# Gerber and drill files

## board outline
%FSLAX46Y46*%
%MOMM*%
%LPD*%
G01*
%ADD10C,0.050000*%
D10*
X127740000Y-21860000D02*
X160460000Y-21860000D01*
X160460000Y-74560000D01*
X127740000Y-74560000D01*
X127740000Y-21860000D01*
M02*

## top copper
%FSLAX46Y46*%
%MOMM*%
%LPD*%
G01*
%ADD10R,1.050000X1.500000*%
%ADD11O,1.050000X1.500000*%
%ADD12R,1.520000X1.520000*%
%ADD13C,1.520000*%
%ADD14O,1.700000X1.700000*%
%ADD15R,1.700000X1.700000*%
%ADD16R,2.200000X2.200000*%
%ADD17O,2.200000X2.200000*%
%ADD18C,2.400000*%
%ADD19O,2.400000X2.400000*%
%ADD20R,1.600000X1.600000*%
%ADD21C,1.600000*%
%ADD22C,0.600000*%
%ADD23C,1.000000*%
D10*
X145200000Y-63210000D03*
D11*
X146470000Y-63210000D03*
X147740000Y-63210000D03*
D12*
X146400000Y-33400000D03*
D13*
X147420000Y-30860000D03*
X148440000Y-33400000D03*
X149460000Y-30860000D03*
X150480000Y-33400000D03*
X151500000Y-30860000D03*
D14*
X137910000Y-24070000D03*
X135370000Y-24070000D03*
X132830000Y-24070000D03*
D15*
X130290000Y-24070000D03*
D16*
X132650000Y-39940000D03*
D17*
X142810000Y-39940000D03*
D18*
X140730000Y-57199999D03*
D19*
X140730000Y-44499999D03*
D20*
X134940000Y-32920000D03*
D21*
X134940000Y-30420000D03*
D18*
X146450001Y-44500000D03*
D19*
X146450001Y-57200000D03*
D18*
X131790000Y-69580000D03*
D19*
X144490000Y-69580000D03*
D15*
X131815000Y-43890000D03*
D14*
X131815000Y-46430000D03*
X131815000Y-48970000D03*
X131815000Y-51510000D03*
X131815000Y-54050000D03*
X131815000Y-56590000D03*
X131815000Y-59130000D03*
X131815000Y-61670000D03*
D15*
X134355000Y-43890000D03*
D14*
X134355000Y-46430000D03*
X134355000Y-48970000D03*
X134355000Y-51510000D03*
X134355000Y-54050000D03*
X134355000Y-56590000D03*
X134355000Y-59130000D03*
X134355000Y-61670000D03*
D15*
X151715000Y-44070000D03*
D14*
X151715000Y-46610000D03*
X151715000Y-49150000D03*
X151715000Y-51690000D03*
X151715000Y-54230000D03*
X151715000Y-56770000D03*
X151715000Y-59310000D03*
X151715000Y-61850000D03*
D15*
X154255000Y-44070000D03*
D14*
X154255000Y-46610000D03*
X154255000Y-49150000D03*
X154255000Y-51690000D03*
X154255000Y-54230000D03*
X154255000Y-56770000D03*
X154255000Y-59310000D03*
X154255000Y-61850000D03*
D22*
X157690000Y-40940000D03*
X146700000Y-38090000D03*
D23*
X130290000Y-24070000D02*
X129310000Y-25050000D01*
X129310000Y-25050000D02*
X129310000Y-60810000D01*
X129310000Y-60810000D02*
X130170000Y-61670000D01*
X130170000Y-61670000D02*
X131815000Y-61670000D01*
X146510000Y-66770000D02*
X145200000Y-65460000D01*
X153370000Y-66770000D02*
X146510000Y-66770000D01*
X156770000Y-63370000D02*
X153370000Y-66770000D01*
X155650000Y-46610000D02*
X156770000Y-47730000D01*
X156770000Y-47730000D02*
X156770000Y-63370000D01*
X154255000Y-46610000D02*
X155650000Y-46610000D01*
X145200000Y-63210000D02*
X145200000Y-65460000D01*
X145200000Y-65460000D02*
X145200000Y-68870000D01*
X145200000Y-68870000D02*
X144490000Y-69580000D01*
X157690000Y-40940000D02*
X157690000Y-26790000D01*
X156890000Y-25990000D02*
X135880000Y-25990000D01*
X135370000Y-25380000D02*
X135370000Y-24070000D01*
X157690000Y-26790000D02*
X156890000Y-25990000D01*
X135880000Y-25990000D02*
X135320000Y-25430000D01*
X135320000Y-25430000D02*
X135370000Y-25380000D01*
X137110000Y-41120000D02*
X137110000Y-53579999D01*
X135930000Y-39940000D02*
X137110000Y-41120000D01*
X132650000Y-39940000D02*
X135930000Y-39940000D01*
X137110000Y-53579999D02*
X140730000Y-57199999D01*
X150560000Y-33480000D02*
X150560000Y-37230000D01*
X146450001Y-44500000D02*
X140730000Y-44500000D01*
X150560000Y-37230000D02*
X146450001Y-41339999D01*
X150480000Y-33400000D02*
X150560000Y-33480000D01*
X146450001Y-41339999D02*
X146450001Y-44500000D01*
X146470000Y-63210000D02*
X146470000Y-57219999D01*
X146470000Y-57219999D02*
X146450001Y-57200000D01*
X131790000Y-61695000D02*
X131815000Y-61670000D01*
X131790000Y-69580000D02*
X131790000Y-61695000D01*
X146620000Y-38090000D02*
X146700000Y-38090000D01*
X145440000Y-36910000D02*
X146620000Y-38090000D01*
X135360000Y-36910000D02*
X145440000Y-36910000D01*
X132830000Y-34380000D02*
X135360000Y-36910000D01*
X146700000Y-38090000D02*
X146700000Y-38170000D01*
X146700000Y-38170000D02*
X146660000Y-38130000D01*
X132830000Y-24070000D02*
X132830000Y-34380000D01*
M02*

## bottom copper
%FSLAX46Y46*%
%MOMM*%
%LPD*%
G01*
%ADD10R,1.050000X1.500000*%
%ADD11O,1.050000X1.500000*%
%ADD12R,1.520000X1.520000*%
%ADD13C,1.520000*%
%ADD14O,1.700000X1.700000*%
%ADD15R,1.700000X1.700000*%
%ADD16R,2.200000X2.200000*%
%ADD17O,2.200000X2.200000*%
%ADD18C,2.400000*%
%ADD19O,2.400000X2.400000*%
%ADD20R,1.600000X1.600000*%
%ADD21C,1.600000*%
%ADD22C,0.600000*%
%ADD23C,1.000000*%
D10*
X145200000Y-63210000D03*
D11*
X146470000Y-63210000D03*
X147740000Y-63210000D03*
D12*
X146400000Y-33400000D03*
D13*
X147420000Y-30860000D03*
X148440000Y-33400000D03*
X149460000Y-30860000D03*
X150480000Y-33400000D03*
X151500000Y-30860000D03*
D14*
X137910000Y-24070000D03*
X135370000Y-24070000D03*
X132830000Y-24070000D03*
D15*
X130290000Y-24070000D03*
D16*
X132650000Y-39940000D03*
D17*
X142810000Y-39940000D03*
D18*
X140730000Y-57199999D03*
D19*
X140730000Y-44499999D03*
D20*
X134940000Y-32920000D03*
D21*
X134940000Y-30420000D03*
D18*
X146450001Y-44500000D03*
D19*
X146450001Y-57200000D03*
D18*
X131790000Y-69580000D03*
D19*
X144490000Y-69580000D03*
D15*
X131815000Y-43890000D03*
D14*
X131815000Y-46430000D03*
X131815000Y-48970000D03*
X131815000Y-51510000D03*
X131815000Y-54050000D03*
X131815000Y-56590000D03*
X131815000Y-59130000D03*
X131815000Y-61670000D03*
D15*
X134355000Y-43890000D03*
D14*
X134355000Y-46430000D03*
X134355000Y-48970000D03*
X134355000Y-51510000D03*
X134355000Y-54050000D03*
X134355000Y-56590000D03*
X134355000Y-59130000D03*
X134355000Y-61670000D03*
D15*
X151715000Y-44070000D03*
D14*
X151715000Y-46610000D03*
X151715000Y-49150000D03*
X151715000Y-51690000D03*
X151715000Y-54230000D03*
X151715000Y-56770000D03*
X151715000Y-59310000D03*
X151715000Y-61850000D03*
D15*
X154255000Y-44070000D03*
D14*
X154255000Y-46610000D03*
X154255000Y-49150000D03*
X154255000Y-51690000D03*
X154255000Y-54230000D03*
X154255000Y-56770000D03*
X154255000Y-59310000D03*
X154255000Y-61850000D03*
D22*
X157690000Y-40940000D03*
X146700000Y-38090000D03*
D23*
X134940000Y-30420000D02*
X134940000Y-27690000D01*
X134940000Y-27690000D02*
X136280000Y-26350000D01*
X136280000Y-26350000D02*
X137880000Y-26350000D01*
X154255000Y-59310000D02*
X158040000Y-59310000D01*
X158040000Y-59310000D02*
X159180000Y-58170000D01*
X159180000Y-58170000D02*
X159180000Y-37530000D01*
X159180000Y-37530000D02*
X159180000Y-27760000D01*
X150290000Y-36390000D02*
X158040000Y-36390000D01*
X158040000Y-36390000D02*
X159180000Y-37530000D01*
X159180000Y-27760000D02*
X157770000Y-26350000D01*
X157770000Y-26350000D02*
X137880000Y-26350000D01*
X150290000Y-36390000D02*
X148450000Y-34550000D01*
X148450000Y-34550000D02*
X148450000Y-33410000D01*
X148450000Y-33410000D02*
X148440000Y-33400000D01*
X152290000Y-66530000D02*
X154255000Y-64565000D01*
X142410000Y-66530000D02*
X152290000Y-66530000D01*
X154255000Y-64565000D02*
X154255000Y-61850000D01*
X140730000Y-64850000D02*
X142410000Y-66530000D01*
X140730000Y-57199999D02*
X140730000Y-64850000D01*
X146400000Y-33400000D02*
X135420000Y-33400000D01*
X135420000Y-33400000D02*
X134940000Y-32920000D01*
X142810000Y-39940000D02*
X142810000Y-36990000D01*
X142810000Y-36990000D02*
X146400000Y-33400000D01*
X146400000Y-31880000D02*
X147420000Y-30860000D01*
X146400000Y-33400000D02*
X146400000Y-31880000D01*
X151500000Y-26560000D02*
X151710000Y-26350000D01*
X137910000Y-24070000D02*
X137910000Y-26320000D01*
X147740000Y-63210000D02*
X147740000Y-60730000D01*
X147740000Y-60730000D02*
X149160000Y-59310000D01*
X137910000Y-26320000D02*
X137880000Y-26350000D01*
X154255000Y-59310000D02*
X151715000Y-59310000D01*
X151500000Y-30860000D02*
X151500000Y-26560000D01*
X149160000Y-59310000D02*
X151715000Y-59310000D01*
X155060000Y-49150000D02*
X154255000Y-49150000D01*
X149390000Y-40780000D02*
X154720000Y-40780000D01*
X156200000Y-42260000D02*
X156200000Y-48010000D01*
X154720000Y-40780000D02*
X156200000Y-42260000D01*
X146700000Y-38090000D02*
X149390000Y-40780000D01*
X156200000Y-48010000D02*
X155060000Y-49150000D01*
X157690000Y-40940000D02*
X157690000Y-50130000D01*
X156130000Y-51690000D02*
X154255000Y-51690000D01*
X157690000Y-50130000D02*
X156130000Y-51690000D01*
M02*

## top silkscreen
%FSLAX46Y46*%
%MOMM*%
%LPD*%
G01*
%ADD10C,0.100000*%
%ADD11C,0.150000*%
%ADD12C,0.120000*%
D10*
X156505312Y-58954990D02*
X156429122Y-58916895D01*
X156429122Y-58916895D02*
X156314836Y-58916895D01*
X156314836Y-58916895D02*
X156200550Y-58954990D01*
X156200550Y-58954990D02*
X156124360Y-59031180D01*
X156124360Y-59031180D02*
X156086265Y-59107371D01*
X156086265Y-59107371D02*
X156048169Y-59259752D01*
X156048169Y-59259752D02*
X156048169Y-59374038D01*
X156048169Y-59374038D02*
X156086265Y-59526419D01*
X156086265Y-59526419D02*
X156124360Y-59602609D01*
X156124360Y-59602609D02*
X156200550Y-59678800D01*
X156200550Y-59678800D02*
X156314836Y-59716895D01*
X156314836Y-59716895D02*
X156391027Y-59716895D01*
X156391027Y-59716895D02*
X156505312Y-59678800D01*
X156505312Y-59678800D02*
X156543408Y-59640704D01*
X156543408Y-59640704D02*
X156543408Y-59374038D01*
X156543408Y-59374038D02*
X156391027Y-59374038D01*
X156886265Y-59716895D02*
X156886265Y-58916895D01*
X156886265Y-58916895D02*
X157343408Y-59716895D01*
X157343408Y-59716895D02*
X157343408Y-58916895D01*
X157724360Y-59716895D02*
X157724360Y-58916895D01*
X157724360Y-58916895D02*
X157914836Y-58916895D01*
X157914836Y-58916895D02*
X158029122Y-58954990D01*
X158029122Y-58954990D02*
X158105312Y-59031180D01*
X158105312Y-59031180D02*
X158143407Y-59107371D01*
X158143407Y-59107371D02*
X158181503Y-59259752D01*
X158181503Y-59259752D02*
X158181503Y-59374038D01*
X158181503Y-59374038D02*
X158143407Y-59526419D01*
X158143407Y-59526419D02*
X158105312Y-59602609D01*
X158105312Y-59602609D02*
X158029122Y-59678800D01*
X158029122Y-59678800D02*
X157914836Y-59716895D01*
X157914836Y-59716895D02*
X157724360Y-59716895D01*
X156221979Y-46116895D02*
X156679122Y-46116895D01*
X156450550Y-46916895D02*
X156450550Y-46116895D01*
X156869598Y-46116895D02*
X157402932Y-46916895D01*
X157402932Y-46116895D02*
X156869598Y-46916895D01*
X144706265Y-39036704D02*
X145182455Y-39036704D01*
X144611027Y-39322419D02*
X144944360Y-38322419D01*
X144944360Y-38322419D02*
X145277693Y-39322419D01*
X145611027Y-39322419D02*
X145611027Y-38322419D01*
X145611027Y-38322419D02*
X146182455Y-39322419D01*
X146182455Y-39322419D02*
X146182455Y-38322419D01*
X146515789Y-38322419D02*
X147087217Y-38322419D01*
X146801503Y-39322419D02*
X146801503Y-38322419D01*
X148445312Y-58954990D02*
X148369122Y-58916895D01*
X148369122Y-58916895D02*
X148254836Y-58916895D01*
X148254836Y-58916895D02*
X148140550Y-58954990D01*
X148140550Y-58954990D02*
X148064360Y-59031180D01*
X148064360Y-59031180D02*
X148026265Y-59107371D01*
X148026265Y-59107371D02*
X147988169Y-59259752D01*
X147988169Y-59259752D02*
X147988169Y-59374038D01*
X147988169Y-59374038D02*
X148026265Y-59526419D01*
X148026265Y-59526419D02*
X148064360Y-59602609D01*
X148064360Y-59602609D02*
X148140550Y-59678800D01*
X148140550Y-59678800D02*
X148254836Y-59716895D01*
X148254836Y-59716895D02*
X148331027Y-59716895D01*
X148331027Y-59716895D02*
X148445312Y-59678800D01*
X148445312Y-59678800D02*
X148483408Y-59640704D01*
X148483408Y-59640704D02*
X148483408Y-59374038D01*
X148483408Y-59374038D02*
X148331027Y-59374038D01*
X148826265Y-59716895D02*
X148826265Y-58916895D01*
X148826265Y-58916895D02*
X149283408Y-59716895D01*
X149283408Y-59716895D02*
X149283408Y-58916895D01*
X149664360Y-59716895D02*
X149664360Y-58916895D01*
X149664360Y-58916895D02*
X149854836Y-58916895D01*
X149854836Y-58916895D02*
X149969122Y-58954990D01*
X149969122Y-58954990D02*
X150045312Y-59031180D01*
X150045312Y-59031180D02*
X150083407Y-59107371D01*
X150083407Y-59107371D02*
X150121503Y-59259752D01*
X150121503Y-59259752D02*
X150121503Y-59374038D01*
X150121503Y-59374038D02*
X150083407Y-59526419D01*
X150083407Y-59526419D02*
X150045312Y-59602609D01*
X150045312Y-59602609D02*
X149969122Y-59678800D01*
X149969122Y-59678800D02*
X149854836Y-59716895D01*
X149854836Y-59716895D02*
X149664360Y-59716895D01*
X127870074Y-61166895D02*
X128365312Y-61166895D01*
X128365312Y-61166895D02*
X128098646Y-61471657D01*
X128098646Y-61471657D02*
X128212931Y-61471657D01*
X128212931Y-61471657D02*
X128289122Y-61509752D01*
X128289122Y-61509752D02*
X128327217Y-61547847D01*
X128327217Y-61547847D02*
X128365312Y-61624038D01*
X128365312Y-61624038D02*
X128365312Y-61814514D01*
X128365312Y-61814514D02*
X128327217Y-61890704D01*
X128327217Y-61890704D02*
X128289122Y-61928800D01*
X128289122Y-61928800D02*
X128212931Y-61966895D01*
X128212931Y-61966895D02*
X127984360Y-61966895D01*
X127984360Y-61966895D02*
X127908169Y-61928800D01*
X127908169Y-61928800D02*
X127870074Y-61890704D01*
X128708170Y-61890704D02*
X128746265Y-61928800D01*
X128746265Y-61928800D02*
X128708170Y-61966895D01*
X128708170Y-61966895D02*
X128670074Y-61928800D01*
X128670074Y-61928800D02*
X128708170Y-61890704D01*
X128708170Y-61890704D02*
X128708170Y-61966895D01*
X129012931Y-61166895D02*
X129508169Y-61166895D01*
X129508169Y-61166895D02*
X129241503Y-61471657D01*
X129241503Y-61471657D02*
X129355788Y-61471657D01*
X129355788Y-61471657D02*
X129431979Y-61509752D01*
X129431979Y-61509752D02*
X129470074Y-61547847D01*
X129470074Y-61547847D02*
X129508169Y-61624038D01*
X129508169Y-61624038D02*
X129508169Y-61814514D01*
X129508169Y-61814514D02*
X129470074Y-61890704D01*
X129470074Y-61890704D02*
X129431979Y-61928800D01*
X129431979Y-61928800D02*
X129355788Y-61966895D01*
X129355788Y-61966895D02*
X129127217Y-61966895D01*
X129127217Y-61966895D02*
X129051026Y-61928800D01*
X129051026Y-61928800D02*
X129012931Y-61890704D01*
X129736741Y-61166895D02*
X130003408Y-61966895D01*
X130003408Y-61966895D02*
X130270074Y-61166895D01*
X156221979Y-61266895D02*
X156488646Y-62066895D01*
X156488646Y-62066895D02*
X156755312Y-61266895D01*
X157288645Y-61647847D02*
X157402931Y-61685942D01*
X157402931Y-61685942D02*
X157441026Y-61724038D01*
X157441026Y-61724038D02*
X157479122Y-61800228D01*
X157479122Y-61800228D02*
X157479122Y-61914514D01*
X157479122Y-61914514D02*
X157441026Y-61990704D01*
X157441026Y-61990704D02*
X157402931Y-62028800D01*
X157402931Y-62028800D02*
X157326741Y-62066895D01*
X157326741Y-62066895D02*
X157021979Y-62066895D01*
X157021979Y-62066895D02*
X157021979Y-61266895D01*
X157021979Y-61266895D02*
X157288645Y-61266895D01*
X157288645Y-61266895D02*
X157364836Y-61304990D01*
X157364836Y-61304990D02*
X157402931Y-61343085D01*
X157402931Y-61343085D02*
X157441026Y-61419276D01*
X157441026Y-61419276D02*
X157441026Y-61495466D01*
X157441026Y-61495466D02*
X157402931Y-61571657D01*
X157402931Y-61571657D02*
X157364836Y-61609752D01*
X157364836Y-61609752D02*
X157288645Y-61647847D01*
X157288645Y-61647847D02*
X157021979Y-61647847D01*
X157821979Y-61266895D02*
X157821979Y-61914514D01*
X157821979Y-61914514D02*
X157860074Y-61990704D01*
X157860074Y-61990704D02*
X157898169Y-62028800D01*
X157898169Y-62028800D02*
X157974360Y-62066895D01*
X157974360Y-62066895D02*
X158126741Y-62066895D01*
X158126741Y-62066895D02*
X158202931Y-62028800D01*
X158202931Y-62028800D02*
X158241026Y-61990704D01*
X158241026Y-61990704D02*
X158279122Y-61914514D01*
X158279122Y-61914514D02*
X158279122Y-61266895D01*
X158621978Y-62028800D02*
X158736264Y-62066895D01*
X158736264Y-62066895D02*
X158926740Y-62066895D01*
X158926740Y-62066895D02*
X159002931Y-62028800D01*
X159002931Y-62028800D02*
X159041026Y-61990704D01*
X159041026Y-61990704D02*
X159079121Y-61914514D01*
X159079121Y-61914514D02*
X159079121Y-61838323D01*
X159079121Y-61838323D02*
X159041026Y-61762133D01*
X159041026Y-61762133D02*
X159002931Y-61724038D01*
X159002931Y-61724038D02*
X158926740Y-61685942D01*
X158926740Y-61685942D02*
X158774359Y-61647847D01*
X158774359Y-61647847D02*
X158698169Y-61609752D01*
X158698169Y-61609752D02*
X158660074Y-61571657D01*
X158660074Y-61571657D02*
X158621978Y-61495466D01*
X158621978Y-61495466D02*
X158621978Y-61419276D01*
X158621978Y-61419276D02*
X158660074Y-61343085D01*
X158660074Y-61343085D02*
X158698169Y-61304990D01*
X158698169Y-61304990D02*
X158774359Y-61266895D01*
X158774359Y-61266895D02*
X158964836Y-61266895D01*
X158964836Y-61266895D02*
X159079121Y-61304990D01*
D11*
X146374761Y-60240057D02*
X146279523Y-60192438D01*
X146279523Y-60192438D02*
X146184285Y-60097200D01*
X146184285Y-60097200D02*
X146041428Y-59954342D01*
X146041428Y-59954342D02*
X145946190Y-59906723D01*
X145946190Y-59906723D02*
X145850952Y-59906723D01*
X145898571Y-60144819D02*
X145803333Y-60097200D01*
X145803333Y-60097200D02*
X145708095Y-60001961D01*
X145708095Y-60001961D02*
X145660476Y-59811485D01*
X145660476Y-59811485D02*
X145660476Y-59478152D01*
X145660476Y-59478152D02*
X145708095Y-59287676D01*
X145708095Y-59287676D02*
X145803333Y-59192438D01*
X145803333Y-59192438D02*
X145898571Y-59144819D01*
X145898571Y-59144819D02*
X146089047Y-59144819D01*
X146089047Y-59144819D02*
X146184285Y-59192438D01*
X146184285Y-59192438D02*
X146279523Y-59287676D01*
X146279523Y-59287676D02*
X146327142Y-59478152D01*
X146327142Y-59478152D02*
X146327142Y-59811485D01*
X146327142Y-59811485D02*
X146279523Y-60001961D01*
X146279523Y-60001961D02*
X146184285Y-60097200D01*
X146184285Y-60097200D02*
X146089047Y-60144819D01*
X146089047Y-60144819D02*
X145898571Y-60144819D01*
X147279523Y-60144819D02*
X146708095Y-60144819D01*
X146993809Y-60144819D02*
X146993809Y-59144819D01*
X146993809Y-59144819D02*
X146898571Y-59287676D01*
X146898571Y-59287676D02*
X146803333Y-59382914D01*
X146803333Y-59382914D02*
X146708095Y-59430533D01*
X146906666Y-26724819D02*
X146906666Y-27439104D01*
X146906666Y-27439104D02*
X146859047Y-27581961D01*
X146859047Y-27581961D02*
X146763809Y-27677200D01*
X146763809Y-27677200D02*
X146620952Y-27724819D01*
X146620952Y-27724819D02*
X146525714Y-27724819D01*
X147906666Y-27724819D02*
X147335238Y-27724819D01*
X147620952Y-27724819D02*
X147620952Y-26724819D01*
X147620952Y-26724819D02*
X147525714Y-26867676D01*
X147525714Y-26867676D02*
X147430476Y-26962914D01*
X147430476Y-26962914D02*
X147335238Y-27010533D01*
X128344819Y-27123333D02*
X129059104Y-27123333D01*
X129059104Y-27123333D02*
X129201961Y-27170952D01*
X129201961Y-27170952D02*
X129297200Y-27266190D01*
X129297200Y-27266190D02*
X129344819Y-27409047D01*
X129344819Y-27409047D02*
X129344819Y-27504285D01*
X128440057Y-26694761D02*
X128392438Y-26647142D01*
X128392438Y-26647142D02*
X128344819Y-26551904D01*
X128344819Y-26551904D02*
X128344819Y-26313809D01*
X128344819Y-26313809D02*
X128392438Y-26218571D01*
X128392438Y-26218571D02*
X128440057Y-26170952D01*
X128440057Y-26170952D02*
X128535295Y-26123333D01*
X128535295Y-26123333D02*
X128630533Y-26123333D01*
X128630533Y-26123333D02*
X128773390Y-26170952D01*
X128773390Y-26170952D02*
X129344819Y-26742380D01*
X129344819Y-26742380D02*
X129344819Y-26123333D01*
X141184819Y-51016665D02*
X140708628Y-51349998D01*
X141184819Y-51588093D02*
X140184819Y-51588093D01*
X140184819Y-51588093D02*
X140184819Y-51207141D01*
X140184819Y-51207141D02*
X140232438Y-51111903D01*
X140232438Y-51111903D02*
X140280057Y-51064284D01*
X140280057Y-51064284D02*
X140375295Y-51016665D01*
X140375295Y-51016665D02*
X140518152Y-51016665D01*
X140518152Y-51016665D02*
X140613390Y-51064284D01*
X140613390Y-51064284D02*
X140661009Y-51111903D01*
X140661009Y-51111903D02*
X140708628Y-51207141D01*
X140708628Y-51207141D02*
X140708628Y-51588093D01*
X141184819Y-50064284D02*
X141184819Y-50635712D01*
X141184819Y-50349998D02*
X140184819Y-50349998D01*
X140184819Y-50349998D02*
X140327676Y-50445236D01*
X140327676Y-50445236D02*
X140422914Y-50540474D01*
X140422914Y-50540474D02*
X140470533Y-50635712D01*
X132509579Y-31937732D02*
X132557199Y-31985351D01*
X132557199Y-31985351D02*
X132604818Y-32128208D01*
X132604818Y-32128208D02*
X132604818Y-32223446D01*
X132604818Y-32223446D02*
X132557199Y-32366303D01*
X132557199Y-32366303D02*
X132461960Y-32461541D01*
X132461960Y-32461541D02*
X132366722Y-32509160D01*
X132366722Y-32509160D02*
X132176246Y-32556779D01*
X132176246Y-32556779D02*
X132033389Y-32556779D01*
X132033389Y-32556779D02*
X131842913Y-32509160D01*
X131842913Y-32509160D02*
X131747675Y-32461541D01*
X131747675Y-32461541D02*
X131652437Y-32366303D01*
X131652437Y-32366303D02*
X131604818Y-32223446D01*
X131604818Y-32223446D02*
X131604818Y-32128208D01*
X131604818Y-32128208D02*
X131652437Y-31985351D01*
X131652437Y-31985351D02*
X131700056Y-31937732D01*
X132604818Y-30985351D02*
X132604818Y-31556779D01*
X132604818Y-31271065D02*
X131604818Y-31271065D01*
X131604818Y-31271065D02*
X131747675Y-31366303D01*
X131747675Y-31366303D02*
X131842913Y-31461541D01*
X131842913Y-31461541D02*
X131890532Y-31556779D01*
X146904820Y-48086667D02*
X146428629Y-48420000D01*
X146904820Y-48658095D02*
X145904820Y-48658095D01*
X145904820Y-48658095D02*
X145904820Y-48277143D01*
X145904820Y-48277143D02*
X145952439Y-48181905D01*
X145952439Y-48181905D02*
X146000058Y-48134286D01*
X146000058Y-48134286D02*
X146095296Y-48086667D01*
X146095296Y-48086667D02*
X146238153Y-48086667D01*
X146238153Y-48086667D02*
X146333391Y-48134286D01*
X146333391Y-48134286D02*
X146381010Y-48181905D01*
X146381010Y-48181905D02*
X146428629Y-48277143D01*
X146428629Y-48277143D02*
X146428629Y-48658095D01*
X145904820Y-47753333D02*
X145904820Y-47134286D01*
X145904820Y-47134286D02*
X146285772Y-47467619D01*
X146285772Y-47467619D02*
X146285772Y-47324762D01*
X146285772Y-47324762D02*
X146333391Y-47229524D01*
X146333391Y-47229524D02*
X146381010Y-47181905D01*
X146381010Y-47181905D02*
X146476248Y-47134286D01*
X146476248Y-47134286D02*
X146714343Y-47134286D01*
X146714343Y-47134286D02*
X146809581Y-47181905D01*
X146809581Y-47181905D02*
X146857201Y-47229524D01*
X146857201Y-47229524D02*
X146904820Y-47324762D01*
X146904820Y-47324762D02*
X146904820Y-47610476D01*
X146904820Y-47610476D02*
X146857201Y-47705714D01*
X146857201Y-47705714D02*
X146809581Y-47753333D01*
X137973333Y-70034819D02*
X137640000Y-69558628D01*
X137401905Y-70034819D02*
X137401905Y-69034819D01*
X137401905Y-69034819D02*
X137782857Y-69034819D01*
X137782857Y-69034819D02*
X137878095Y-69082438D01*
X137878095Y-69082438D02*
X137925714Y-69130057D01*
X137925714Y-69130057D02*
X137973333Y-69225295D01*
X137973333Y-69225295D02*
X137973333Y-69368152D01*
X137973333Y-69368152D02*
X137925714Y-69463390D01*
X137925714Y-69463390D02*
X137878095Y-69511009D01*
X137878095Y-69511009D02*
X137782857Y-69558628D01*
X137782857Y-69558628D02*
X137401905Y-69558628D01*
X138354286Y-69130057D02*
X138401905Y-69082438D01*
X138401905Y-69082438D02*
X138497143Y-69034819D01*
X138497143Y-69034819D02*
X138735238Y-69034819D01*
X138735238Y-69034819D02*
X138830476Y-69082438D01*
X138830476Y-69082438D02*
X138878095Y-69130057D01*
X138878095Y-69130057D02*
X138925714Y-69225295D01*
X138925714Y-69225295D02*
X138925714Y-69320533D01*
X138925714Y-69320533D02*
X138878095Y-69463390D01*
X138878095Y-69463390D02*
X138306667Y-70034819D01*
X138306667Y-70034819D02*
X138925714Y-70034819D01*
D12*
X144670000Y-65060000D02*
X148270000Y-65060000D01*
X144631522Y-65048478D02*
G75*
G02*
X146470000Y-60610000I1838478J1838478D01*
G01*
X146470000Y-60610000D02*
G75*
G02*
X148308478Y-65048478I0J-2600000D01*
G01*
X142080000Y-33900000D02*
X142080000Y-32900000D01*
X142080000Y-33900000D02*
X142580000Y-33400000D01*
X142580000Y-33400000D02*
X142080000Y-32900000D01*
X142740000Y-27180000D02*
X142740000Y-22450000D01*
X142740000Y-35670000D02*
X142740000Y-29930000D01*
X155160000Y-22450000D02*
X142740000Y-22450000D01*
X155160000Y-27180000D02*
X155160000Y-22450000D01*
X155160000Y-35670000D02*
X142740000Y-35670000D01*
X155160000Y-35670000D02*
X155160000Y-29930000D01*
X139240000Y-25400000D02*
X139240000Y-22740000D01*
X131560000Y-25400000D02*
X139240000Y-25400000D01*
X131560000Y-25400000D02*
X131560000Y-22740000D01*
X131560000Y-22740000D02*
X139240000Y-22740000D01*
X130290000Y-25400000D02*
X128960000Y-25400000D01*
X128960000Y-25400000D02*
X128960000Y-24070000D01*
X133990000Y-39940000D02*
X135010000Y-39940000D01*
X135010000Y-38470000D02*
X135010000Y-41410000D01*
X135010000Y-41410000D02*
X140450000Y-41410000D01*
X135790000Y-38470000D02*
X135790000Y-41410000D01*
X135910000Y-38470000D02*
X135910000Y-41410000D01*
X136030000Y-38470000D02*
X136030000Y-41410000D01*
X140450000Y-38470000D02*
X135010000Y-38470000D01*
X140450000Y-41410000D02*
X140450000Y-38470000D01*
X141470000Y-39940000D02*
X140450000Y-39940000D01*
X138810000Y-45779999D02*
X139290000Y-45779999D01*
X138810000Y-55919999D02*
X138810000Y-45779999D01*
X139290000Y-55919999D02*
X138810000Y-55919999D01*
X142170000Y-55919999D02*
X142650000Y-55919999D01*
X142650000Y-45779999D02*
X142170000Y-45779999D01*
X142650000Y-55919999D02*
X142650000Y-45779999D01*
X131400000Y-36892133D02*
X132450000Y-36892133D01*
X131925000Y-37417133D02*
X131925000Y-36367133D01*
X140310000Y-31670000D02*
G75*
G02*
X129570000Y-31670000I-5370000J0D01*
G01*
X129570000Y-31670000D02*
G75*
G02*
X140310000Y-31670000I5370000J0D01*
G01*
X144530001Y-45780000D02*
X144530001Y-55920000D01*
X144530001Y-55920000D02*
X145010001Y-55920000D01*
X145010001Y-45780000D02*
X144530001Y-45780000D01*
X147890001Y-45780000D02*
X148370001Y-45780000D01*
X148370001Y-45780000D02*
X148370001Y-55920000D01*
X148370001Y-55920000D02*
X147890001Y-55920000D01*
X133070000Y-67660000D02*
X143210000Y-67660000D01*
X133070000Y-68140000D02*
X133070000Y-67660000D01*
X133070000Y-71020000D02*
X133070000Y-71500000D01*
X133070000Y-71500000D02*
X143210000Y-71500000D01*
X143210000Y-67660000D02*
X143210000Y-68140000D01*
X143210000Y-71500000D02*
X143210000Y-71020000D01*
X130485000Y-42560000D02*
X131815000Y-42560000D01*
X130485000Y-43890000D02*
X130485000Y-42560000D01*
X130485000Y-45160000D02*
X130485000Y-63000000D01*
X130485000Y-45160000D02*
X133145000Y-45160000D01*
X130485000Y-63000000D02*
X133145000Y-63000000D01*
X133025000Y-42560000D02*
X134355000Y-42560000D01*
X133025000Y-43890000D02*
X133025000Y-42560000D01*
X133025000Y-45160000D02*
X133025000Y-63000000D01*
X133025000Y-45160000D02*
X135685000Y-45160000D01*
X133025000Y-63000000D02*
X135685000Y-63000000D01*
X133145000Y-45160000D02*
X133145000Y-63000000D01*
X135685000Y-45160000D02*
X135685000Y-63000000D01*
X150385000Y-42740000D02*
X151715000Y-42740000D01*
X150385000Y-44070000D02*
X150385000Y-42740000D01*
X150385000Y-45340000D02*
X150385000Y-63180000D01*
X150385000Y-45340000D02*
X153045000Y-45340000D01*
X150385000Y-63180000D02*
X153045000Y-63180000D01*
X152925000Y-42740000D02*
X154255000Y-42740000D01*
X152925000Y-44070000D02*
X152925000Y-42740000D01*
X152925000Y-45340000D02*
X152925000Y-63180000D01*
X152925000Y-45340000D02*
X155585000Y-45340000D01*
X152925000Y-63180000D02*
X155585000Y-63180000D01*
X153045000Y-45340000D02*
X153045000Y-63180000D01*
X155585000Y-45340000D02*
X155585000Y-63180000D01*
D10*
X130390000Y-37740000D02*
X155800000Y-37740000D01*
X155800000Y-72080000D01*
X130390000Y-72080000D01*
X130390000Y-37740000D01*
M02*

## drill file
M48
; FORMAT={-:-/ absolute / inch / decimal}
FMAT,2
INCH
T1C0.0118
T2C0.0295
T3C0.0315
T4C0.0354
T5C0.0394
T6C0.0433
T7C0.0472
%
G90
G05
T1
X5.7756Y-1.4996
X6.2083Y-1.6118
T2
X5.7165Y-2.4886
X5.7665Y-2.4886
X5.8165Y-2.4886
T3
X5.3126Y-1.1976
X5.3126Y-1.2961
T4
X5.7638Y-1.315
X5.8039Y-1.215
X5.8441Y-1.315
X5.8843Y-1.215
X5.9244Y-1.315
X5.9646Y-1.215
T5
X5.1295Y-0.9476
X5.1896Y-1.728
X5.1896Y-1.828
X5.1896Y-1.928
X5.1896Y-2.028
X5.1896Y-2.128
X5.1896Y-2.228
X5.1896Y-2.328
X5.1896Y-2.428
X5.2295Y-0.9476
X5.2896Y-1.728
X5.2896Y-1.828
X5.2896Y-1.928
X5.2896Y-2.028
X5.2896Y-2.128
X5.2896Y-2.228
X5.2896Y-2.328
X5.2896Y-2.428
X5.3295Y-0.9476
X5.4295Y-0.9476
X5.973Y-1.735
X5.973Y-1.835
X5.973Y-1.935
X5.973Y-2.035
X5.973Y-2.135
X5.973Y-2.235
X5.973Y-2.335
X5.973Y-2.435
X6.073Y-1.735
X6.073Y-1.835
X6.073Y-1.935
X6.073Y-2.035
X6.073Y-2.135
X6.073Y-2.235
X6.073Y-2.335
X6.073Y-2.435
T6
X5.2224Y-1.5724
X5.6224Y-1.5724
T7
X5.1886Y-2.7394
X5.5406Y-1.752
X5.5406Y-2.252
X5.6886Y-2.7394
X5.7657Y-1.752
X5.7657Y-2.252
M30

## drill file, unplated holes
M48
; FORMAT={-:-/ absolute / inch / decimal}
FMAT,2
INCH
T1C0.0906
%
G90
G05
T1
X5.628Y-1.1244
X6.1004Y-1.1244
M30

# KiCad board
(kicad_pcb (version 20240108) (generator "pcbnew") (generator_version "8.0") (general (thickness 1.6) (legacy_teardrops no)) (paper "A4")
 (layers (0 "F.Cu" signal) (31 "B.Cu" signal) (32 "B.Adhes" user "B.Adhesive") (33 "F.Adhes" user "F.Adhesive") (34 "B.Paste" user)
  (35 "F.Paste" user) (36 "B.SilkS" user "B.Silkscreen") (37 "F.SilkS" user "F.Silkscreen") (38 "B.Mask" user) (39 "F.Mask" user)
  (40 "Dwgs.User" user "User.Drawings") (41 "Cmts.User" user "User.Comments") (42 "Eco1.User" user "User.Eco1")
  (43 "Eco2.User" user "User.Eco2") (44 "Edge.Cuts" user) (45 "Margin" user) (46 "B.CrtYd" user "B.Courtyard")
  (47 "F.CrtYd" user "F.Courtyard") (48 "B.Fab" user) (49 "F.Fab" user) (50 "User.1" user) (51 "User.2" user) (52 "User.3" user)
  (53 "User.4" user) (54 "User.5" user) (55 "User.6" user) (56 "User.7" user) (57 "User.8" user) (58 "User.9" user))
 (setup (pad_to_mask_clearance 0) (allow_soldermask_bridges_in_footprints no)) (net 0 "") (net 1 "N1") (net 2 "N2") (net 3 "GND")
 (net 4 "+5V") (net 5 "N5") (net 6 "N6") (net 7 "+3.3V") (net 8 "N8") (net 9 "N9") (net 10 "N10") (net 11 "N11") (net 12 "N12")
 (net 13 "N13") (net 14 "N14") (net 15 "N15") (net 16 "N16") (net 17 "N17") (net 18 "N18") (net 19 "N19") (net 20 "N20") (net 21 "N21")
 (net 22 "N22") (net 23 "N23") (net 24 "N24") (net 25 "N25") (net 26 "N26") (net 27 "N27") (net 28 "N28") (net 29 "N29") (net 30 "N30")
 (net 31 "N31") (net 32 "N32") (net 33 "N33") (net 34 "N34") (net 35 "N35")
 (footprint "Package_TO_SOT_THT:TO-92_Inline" (layer "F.Cu") (at 145.2 63.21)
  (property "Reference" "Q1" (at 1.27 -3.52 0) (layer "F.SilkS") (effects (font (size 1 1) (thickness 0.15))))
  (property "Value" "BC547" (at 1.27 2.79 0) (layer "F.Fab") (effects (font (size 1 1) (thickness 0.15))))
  (fp_line (start -0.53 1.85) (end 3.07 1.85) (stroke (width 0.12) (type solid)) (layer "F.SilkS"))
  (fp_arc (start -0.568478 1.838478) (mid -1.132087 -0.994977) (end 1.27 -2.6) (stroke (width 0.12) (type solid)) (layer "F.SilkS"))
  (fp_arc (start 1.27 -2.6) (mid 3.672087 -0.994977) (end 3.108478 1.838478) (stroke (width 0.12) (type solid)) (layer "F.SilkS"))
  (pad "1" thru_hole rect (at 0 0) (size 1.05 1.5) (drill 0.75) (layers "*.Cu" "*.Mask") (remove_unused_layers no) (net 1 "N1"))
  (pad "2" thru_hole oval (at 1.27 0) (size 1.05 1.5) (drill 0.75) (layers "*.Cu" "*.Mask") (remove_unused_layers no) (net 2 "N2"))
  (pad "3" thru_hole oval (at 2.54 0) (size 1.05 1.5) (drill 0.75) (layers "*.Cu" "*.Mask") (remove_unused_layers no) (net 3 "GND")))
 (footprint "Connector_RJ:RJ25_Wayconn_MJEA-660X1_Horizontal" (layer "F.Cu") (at 146.4 33.4 180)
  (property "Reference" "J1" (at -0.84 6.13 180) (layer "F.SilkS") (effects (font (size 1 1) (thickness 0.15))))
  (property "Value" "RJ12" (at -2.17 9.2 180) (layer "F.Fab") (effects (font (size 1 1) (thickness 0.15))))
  (fp_line (start 4.32 -0.5) (end 4.32 0.5) (stroke (width 0.12) (type solid)) (layer "F.SilkS"))
  (fp_line (start 4.32 -0.5) (end 3.82 0) (stroke (width 0.12) (type solid)) (layer "F.SilkS"))
  (fp_line (start 3.82 0) (end 4.32 0.5) (stroke (width 0.12) (type solid)) (layer "F.SilkS"))
  (fp_line (start 3.66 6.22) (end 3.66 10.95) (stroke (width 0.12) (type solid)) (layer "F.SilkS"))
  (fp_line (start 3.66 -2.27) (end 3.66 3.47) (stroke (width 0.12) (type solid)) (layer "F.SilkS"))
  (fp_line (start -8.76 10.95) (end 3.66 10.95) (stroke (width 0.12) (type solid)) (layer "F.SilkS"))
  (fp_line (start -8.76 6.22) (end -8.76 10.95) (stroke (width 0.12) (type solid)) (layer "F.SilkS"))
  (fp_line (start -8.76 -2.27) (end 3.66 -2.27) (stroke (width 0.12) (type solid)) (layer "F.SilkS"))
  (fp_line (start -8.76 -2.27) (end -8.76 3.47) (stroke (width 0.12) (type solid)) (layer "F.SilkS"))
  (pad "" np_thru_hole circle (at -8.55 4.84 180) (size 2.3 2.3) (drill 2.3) (layers "*.Cu" "*.Mask"))
  (pad "" np_thru_hole circle (at 3.45 4.84 180) (size 2.3 2.3) (drill 2.3) (layers "*.Cu" "*.Mask"))
  (pad "1" thru_hole rect (at 0 0 180) (size 1.52 1.52) (drill 0.9) (layers "*.Cu" "*.Mask") (remove_unused_layers no) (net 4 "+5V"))
  (pad "2" thru_hole circle (at -1.02 2.54 180) (size 1.52 1.52) (drill 0.9) (layers "*.Cu" "*.Mask") (remove_unused_layers no)
   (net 4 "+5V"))
  (pad "3" thru_hole circle (at -2.04 0 180) (size 1.52 1.52) (drill 0.9) (layers "*.Cu" "*.Mask") (remove_unused_layers no) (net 3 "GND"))
  (pad "4" thru_hole circle (at -3.06 2.54 180) (size 1.52 1.52) (drill 0.9) (layers "*.Cu" "*.Mask") (remove_unused_layers no) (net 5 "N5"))
  (pad "5" thru_hole circle (at -4.08 0 180) (size 1.52 1.52) (drill 0.9) (layers "*.Cu" "*.Mask") (remove_unused_layers no) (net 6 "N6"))
  (pad "6" thru_hole circle (at -5.1 2.54 180) (size 1.52 1.52) (drill 0.9) (layers "*.Cu" "*.Mask") (remove_unused_layers no) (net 3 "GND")))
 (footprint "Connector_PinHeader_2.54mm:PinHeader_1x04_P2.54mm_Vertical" (layer "F.Cu") (at 130.29 24.07 90)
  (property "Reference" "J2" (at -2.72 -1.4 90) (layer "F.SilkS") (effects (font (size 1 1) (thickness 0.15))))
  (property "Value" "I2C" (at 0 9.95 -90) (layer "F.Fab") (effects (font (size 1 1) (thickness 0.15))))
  (fp_line (start -1.33 -1.33) (end 0 -1.33) (stroke (width 0.12) (type solid)) (layer "F.SilkS"))
  (fp_line (start -1.33 0) (end -1.33 -1.33) (stroke (width 0.12) (type solid)) (layer "F.SilkS"))
  (fp_line (start 1.33 1.27) (end 1.33 8.95) (stroke (width 0.12) (type solid)) (layer "F.SilkS"))
  (fp_line (start -1.33 1.27) (end 1.33 1.27) (stroke (width 0.12) (type solid)) (layer "F.SilkS"))
  (fp_line (start -1.33 1.27) (end -1.33 8.95) (stroke (width 0.12) (type solid)) (layer "F.SilkS"))
  (fp_line (start -1.33 8.95) (end 1.33 8.95) (stroke (width 0.12) (type solid)) (layer "F.SilkS"))
  (pad "1" thru_hole rect (at 0 0 90) (size 1.7 1.7) (drill 1) (layers "*.Cu" "*.Mask") (remove_unused_layers no) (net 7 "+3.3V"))
  (pad "2" thru_hole oval (at 0 2.54 90) (size 1.7 1.7) (drill 1) (layers "*.Cu" "*.Mask") (remove_unused_layers no) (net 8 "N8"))
  (pad "3" thru_hole oval (at 0 5.08 90) (size 1.7 1.7) (drill 1) (layers "*.Cu" "*.Mask") (remove_unused_layers no) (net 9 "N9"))
  (pad "4" thru_hole oval (at 0 7.62 90) (size 1.7 1.7) (drill 1) (layers "*.Cu" "*.Mask") (remove_unused_layers no) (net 3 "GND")))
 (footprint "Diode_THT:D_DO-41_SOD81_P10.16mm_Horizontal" (layer "F.Cu") (at 132.65 39.94)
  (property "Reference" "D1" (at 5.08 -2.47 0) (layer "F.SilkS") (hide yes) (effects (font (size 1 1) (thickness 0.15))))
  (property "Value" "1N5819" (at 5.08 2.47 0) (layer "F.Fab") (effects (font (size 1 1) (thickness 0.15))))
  (fp_line (start 1.34 0) (end 2.36 0) (stroke (width 0.12) (type solid)) (layer "F.SilkS"))
  (fp_line (start 2.36 -1.47) (end 2.36 1.47) (stroke (width 0.12) (type solid)) (layer "F.SilkS"))
  (fp_line (start 2.36 1.47) (end 7.8 1.47) (stroke (width 0.12) (type solid)) (layer "F.SilkS"))
  (fp_line (start 3.14 -1.47) (end 3.14 1.47) (stroke (width 0.12) (type solid)) (layer "F.SilkS"))
  (fp_line (start 3.26 -1.47) (end 3.26 1.47) (stroke (width 0.12) (type solid)) (layer "F.SilkS"))
  (fp_line (start 3.38 -1.47) (end 3.38 1.47) (stroke (width 0.12) (type solid)) (layer "F.SilkS"))
  (fp_line (start 7.8 -1.47) (end 2.36 -1.47) (stroke (width 0.12) (type solid)) (layer "F.SilkS"))
  (fp_line (start 7.8 1.47) (end 7.8 -1.47) (stroke (width 0.12) (type solid)) (layer "F.SilkS"))
  (fp_line (start 8.82 0) (end 7.8 0) (stroke (width 0.12) (type solid)) (layer "F.SilkS"))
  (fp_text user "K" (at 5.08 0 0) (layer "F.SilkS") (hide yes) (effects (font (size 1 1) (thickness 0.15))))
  (pad "1" thru_hole rect (at 0 0) (size 2.2 2.2) (drill 1.1) (layers "*.Cu" "*.Mask") (remove_unused_layers no) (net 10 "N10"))
  (pad "2" thru_hole oval (at 10.16 0) (size 2.2 2.2) (drill 1.1) (layers "*.Cu" "*.Mask") (remove_unused_layers no) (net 4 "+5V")))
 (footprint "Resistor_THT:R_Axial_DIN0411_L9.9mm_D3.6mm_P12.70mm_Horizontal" (layer "F.Cu") (at 140.73 57.199999 90)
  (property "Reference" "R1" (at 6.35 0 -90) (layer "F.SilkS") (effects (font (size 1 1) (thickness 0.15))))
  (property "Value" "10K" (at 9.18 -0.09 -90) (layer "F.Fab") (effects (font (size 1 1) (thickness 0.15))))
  (fp_line (start 11.42 -1.92) (end 11.42 -1.44) (stroke (width 0.12) (type solid)) (layer "F.SilkS"))
  (fp_line (start 1.28 -1.92) (end 11.42 -1.92) (stroke (width 0.12) (type solid)) (layer "F.SilkS"))
  (fp_line (start 1.28 -1.44) (end 1.28 -1.92) (stroke (width 0.12) (type solid)) (layer "F.SilkS"))
  (fp_line (start 1.28 1.44) (end 1.28 1.92) (stroke (width 0.12) (type solid)) (layer "F.SilkS"))
  (fp_line (start 11.42 1.92) (end 11.42 1.44) (stroke (width 0.12) (type solid)) (layer "F.SilkS"))
  (fp_line (start 1.28 1.92) (end 11.42 1.92) (stroke (width 0.12) (type solid)) (layer "F.SilkS"))
  (pad "1" thru_hole circle (at 0 0 90) (size 2.4 2.4) (drill 1.2) (layers "*.Cu" "*.Mask") (remove_unused_layers no) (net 10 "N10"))
  (pad "2" thru_hole oval (at 12.7 0 90) (size 2.4 2.4) (drill 1.2) (layers "*.Cu" "*.Mask") (remove_unused_layers no) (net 6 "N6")))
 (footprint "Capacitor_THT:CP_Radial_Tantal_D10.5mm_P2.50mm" (layer "F.Cu") (at 134.94 32.92 90)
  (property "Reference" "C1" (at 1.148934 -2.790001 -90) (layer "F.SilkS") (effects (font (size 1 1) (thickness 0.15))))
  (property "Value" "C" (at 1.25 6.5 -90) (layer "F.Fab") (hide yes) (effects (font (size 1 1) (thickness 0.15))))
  (fp_line (start -3.972133 -3.54) (end -3.972133 -2.49) (stroke (width 0.12) (type solid)) (layer "F.SilkS"))
  (fp_line (start -4.497133 -3.015) (end -3.447133 -3.015) (stroke (width 0.12) (type solid)) (layer "F.SilkS"))
  (fp_circle (center 1.25 0) (end 6.62 0) (stroke (width 0.12) (type solid)) (fill none) (layer "F.SilkS"))
  (pad "1" thru_hole rect (at 0 0 90) (size 1.6 1.6) (drill 0.8) (layers "*.Cu" "*.Mask") (remove_unused_layers no) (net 4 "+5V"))
  (pad "2" thru_hole circle (at 2.5 0 90) (size 1.6 1.6) (drill 0.8) (layers "*.Cu" "*.Mask") (remove_unused_layers no) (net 3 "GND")))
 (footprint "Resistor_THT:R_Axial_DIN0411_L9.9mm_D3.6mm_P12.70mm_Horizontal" (layer "F.Cu") (at 146.450001 44.5 -90)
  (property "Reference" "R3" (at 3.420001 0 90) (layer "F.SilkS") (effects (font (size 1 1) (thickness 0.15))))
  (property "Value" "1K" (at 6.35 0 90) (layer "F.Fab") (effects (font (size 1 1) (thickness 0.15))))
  (fp_line (start 1.28 1.92) (end 11.42 1.92) (stroke (width 0.12) (type solid)) (layer "F.SilkS"))
  (fp_line (start 11.42 1.92) (end 11.42 1.44) (stroke (width 0.12) (type solid)) (layer "F.SilkS"))
  (fp_line (start 1.28 1.44) (end 1.28 1.92) (stroke (width 0.12) (type solid)) (layer "F.SilkS"))
  (fp_line (start 1.28 -1.44) (end 1.28 -1.92) (stroke (width 0.12) (type solid)) (layer "F.SilkS"))
  (fp_line (start 1.28 -1.92) (end 11.42 -1.92) (stroke (width 0.12) (type solid)) (layer "F.SilkS"))
  (fp_line (start 11.42 -1.92) (end 11.42 -1.44) (stroke (width 0.12) (type solid)) (layer "F.SilkS"))
  (pad "1" thru_hole circle (at 0 0 270) (size 2.4 2.4) (drill 1.2) (layers "*.Cu" "*.Mask") (remove_unused_layers no) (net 6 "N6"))
  (pad "2" thru_hole oval (at 12.7 0 270) (size 2.4 2.4) (drill 1.2) (layers "*.Cu" "*.Mask") (remove_unused_layers no) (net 2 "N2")))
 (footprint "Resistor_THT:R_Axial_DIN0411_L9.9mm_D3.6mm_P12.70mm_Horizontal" (layer "F.Cu") (at 131.79 69.58)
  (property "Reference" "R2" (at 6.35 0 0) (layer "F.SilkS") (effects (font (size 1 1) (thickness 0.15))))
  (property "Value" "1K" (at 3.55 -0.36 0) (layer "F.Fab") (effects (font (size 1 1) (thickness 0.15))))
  (fp_line (start 1.28 -1.92) (end 11.42 -1.92) (stroke (width 0.12) (type solid)) (layer "F.SilkS"))
  (fp_line (start 1.28 -1.44) (end 1.28 -1.92) (stroke (width 0.12) (type solid)) (layer "F.SilkS"))
  (fp_line (start 1.28 1.44) (end 1.28 1.92) (stroke (width 0.12) (type solid)) (layer "F.SilkS"))
  (fp_line (start 1.28 1.92) (end 11.42 1.92) (stroke (width 0.12) (type solid)) (layer "F.SilkS"))
  (fp_line (start 11.42 -1.92) (end 11.42 -1.44) (stroke (width 0.12) (type solid)) (layer "F.SilkS"))
  (fp_line (start 11.42 1.92) (end 11.42 1.44) (stroke (width 0.12) (type solid)) (layer "F.SilkS"))
  (pad "1" thru_hole circle (at 0 0) (size 2.4 2.4) (drill 1.2) (layers "*.Cu" "*.Mask") (remove_unused_layers no) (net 7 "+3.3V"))
  (pad "2" thru_hole oval (at 12.7 0) (size 2.4 2.4) (drill 1.2) (layers "*.Cu" "*.Mask") (remove_unused_layers no) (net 1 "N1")))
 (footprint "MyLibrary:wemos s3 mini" (layer "F.Cu") (at 142.785 43.8)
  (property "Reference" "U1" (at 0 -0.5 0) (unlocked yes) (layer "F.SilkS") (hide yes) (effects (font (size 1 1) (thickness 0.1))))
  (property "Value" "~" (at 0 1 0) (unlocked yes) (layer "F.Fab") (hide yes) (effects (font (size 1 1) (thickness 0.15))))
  (fp_line (start -12.3 -1.24) (end -10.97 -1.24) (stroke (width 0.12) (type solid)) (layer "F.SilkS"))
  (fp_line (start -12.3 0.09) (end -12.3 -1.24) (stroke (width 0.12) (type solid)) (layer "F.SilkS"))
  (fp_line (start -12.3 1.36) (end -12.3 19.2) (stroke (width 0.12) (type solid)) (layer "F.SilkS"))
  (fp_line (start -12.3 1.36) (end -9.64 1.36) (stroke (width 0.12) (type solid)) (layer "F.SilkS"))
  (fp_line (start -12.3 19.2) (end -9.64 19.2) (stroke (width 0.12) (type solid)) (layer "F.SilkS"))
  (fp_line (start -9.76 -1.24) (end -8.43 -1.24) (stroke (width 0.12) (type solid)) (layer "F.SilkS"))
  (fp_line (start -9.76 0.09) (end -9.76 -1.24) (stroke (width 0.12) (type solid)) (layer "F.SilkS"))
  (fp_line (start -9.76 1.36) (end -9.76 19.2) (stroke (width 0.12) (type solid)) (layer "F.SilkS"))
  (fp_line (start -9.76 1.36) (end -7.1 1.36) (stroke (width 0.12) (type solid)) (layer "F.SilkS"))
  (fp_line (start -9.76 19.2) (end -7.1 19.2) (stroke (width 0.12) (type solid)) (layer "F.SilkS"))
  (fp_line (start -9.64 1.36) (end -9.64 19.2) (stroke (width 0.12) (type solid)) (layer "F.SilkS"))
  (fp_line (start -7.1 1.36) (end -7.1 19.2) (stroke (width 0.12) (type solid)) (layer "F.SilkS"))
  (fp_line (start 7.6 -1.06) (end 8.93 -1.06) (stroke (width 0.12) (type solid)) (layer "F.SilkS"))
  (fp_line (start 7.6 0.27) (end 7.6 -1.06) (stroke (width 0.12) (type solid)) (layer "F.SilkS"))
  (fp_line (start 7.6 1.54) (end 7.6 19.38) (stroke (width 0.12) (type solid)) (layer "F.SilkS"))
  (fp_line (start 7.6 1.54) (end 10.26 1.54) (stroke (width 0.12) (type solid)) (layer "F.SilkS"))
  (fp_line (start 7.6 19.38) (end 10.26 19.38) (stroke (width 0.12) (type solid)) (layer "F.SilkS"))
  (fp_line (start 10.14 -1.06) (end 11.47 -1.06) (stroke (width 0.12) (type solid)) (layer "F.SilkS"))
  (fp_line (start 10.14 0.27) (end 10.14 -1.06) (stroke (width 0.12) (type solid)) (layer "F.SilkS"))
  (fp_line (start 10.14 1.54) (end 10.14 19.38) (stroke (width 0.12) (type solid)) (layer "F.SilkS"))
  (fp_line (start 10.14 1.54) (end 12.8 1.54) (stroke (width 0.12) (type solid)) (layer "F.SilkS"))
  (fp_line (start 10.14 19.38) (end 12.8 19.38) (stroke (width 0.12) (type solid)) (layer "F.SilkS"))
  (fp_line (start 10.26 1.54) (end 10.26 19.38) (stroke (width 0.12) (type solid)) (layer "F.SilkS"))
  (fp_line (start 12.8 1.54) (end 12.8 19.38) (stroke (width 0.12) (type solid)) (layer "F.SilkS"))
  (fp_rect (start -12.395 -6.06) (end 13.015 28.28) (stroke (width 0.1) (type default)) (fill none) (layer "F.SilkS"))
  (pad "1" thru_hole rect (at -10.97 0.09) (size 1.7 1.7) (drill 1) (layers "*.Cu" "*.Mask") (remove_unused_layers no) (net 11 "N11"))
  (pad "2" thru_hole oval (at -10.97 2.63) (size 1.7 1.7) (drill 1) (layers "*.Cu" "*.Mask") (remove_unused_layers no) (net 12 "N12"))
  (pad "3" thru_hole oval (at -10.97 5.17) (size 1.7 1.7) (drill 1) (layers "*.Cu" "*.Mask") (remove_unused_layers no) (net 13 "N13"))
  (pad "4" thru_hole oval (at -10.97 7.71) (size 1.7 1.7) (drill 1) (layers "*.Cu" "*.Mask") (remove_unused_layers no) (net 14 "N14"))
  (pad "5" thru_hole oval (at -10.97 10.25) (size 1.7 1.7) (drill 1) (layers "*.Cu" "*.Mask") (remove_unused_layers no) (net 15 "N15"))
  (pad "6" thru_hole oval (at -10.97 12.79) (size 1.7 1.7) (drill 1) (layers "*.Cu" "*.Mask") (remove_unused_layers no) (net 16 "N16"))
  (pad "7" thru_hole oval (at -10.97 15.33) (size 1.7 1.7) (drill 1) (layers "*.Cu" "*.Mask") (remove_unused_layers no) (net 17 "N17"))
  (pad "8" thru_hole oval (at -10.97 17.87) (size 1.7 1.7) (drill 1) (layers "*.Cu" "*.Mask") (remove_unused_layers no) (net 7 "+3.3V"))
  (pad "9" thru_hole rect (at -8.43 0.09) (size 1.7 1.7) (drill 1) (layers "*.Cu" "*.Mask") (remove_unused_layers no) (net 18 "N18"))
  (pad "10" thru_hole oval (at -8.43 2.63) (size 1.7 1.7) (drill 1) (layers "*.Cu" "*.Mask") (remove_unused_layers no) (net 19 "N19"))
  (pad "11" thru_hole oval (at -8.43 5.17) (size 1.7 1.7) (drill 1) (layers "*.Cu" "*.Mask") (remove_unused_layers no) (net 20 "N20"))
  (pad "12" thru_hole oval (at -8.43 7.71) (size 1.7 1.7) (drill 1) (layers "*.Cu" "*.Mask") (remove_unused_layers no) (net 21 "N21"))
  (pad "13" thru_hole oval (at -8.43 10.25) (size 1.7 1.7) (drill 1) (layers "*.Cu" "*.Mask") (remove_unused_layers no) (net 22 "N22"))
  (pad "14" thru_hole oval (at -8.43 12.79) (size 1.7 1.7) (drill 1) (layers "*.Cu" "*.Mask") (remove_unused_layers no) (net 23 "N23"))
  (pad "15" thru_hole oval (at -8.43 15.33) (size 1.7 1.7) (drill 1) (layers "*.Cu" "*.Mask") (remove_unused_layers no) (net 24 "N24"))
  (pad "16" thru_hole oval (at -8.43 17.87) (size 1.7 1.7) (drill 1) (layers "*.Cu" "*.Mask") (remove_unused_layers no) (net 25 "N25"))
  (pad "17" thru_hole rect (at 8.93 0.27) (size 1.7 1.7) (drill 1) (layers "*.Cu" "*.Mask") (remove_unused_layers no) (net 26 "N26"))
  (pad "18" thru_hole oval (at 8.93 2.81) (size 1.7 1.7) (drill 1) (layers "*.Cu" "*.Mask") (remove_unused_layers no) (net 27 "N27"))
  (pad "19" thru_hole oval (at 8.93 5.35) (size 1.7 1.7) (drill 1) (layers "*.Cu" "*.Mask") (remove_unused_layers no) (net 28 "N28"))
  (pad "20" thru_hole oval (at 8.93 7.89) (size 1.7 1.7) (drill 1) (layers "*.Cu" "*.Mask") (remove_unused_layers no) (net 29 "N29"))
  (pad "21" thru_hole oval (at 8.93 10.43) (size 1.7 1.7) (drill 1) (layers "*.Cu" "*.Mask") (remove_unused_layers no) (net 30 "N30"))
  (pad "22" thru_hole oval (at 8.93 12.97) (size 1.7 1.7) (drill 1) (layers "*.Cu" "*.Mask") (remove_unused_layers no) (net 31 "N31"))
  (pad "23" thru_hole oval (at 8.93 15.51) (size 1.7 1.7) (drill 1) (layers "*.Cu" "*.Mask") (remove_unused_layers no) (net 3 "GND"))
  (pad "24" thru_hole oval (at 8.93 18.05) (size 1.7 1.7) (drill 1) (layers "*.Cu" "*.Mask") (remove_unused_layers no) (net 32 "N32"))
  (pad "25" thru_hole rect (at 11.47 0.27) (size 1.7 1.7) (drill 1) (layers "*.Cu" "*.Mask") (remove_unused_layers no) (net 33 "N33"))
  (pad "26" thru_hole oval (at 11.47 2.81) (size 1.7 1.7) (drill 1) (layers "*.Cu" "*.Mask") (remove_unused_layers no) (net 1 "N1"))
  (pad "27" thru_hole oval (at 11.47 5.35) (size 1.7 1.7) (drill 1) (layers "*.Cu" "*.Mask") (remove_unused_layers no) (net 8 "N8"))
  (pad "28" thru_hole oval (at 11.47 7.89) (size 1.7 1.7) (drill 1) (layers "*.Cu" "*.Mask") (remove_unused_layers no) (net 9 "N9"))
  (pad "29" thru_hole oval (at 11.47 10.43) (size 1.7 1.7) (drill 1) (layers "*.Cu" "*.Mask") (remove_unused_layers no) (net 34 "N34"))
  (pad "30" thru_hole oval (at 11.47 12.97) (size 1.7 1.7) (drill 1) (layers "*.Cu" "*.Mask") (remove_unused_layers no) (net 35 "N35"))
  (pad "31" thru_hole oval (at 11.47 15.51) (size 1.7 1.7) (drill 1) (layers "*.Cu" "*.Mask") (remove_unused_layers no) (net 3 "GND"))
  (pad "32" thru_hole oval (at 11.47 18.05) (size 1.7 1.7) (drill 1) (layers "*.Cu" "*.Mask") (remove_unused_layers no) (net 10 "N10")))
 (gr_rect (start 127.74 21.86) (end 160.46 74.56) (stroke (width 0.05) (type default)) (fill none) (layer "Edge.Cuts"))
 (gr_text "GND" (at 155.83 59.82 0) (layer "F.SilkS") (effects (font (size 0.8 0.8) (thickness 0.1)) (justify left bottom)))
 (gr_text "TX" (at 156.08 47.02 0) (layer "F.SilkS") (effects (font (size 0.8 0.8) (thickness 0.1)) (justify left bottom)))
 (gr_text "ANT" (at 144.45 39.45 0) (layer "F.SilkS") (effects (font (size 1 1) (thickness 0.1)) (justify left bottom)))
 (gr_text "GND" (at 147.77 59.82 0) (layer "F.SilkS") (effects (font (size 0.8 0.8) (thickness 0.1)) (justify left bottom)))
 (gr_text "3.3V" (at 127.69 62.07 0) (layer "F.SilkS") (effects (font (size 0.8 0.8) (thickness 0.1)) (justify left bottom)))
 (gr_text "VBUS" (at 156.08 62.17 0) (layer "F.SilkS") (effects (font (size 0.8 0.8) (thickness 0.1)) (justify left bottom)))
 (segment (start 137.11 41.12) (end 137.11 53.579999) (width 1) (layer "F.Cu") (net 10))
 (segment (start 135.93 39.94) (end 137.11 41.12) (width 1) (layer "F.Cu") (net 10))
 (segment (start 132.65 39.94) (end 135.93 39.94) (width 1) (layer "F.Cu") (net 10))
 (segment (start 137.11 53.579999) (end 140.73 57.199999) (width 1) (layer "F.Cu") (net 10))
 (segment (start 152.29 66.53) (end 154.255 64.565) (width 1) (layer "B.Cu") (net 10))
 (segment (start 142.41 66.53) (end 152.29 66.53) (width 1) (layer "B.Cu") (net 10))
 (segment (start 154.255 64.565) (end 154.255 61.85) (width 1) (layer "B.Cu") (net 10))
 (segment (start 140.73 64.85) (end 142.41 66.53) (width 1) (layer "B.Cu") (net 10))
 (segment (start 140.73 57.199999) (end 140.73 64.85) (width 1) (layer "B.Cu") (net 10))
 (segment (start 146.4 33.4) (end 135.42 33.4) (width 1) (layer "B.Cu") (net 4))
 (segment (start 135.42 33.4) (end 134.94 32.92) (width 1) (layer "B.Cu") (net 4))
 (segment (start 142.81 39.94) (end 142.81 36.99) (width 1) (layer "B.Cu") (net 4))
 (segment (start 142.81 36.99) (end 146.4 33.4) (width 1) (layer "B.Cu") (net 4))
 (segment (start 146.4 31.88) (end 147.42 30.86) (width 1) (layer "B.Cu") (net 4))
 (segment (start 146.4 33.4) (end 146.4 31.88) (width 1) (layer "B.Cu") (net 4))
 (segment (start 151.5 26.56) (end 151.71 26.35) (width 1) (layer "B.Cu") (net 3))
 (segment (start 154.255 59.31) (end 158.04 59.31) (width 1) (layer "B.Cu") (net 3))
 (segment (start 150.29 36.39) (end 148.45 34.55) (width 1) (layer "B.Cu") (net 3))
 (segment (start 134.94 30.42) (end 134.94 27.69) (width 1) (layer "B.Cu") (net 3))
 (segment (start 148.45 34.55) (end 148.45 33.41) (width 1) (layer "B.Cu") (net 3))
 (segment (start 159.18 58.17) (end 159.18 37.53) (width 1) (layer "B.Cu") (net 3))
 (segment (start 137.91 24.07) (end 137.91 26.32) (width 1) (layer "B.Cu") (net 3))
 (segment (start 158.04 36.39) (end 159.18 37.53) (width 1) (layer "B.Cu") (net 3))
 (segment (start 147.74 63.21) (end 147.74 60.73) (width 1) (layer "B.Cu") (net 3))
 (segment (start 159.18 37.53) (end 159.18 27.76) (width 1) (layer "B.Cu") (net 3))
 (segment (start 147.74 60.73) (end 149.16 59.31) (width 1) (layer "B.Cu") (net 3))
 (segment (start 158.04 59.31) (end 159.18 58.17) (width 1) (layer "B.Cu") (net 3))
 (segment (start 134.94 27.69) (end 136.28 26.35) (width 1) (layer "B.Cu") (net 3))
 (segment (start 137.91 26.32) (end 137.88 26.35) (width 1) (layer "B.Cu") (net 3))
 (segment (start 154.255 59.31) (end 151.715 59.31) (width 1) (layer "B.Cu") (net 3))
 (segment (start 159.18 27.76) (end 157.77 26.35) (width 1) (layer "B.Cu") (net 3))
 (segment (start 136.28 26.35) (end 137.88 26.35) (width 1) (layer "B.Cu") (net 3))
 (segment (start 157.77 26.35) (end 137.88 26.35) (width 1) (layer "B.Cu") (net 3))
 (segment (start 150.29 36.39) (end 158.04 36.39) (width 1) (layer "B.Cu") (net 3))
 (segment (start 151.5 30.86) (end 151.5 26.56) (width 1) (layer "B.Cu") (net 3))
 (segment (start 149.16 59.31) (end 151.715 59.31) (width 1) (layer "B.Cu") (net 3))
 (segment (start 148.45 33.41) (end 148.44 33.4) (width 1) (layer "B.Cu") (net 3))
 (segment (start 150.56 33.48) (end 150.56 37.23) (width 1) (layer "F.Cu") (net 6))
 (segment (start 146.450001 44.5) (end 140.73 44.5) (width 1) (layer "F.Cu") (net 6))
 (segment (start 150.56 37.23) (end 146.450001 41.339999) (width 1) (layer "F.Cu") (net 6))
 (segment (start 150.48 33.4) (end 150.56 33.48) (width 1) (layer "F.Cu") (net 6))
 (segment (start 146.450001 41.339999) (end 146.450001 44.5) (width 1) (layer "F.Cu") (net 6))
 (segment (start 156.77 63.37) (end 153.37 66.77) (width 1) (layer "F.Cu") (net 1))
 (segment (start 145.2 63.21) (end 145.2 65.46) (width 1) (layer "F.Cu") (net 1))
 (segment (start 155.65 46.61) (end 156.77 47.73) (width 1) (layer "F.Cu") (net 1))
 (segment (start 153.37 66.77) (end 146.51 66.77) (width 1) (layer "F.Cu") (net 1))
 (segment (start 145.2 65.46) (end 145.2 68.87) (width 1) (layer "F.Cu") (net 1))
 (segment (start 154.255 46.61) (end 155.65 46.61) (width 1) (layer "F.Cu") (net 1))
 (segment (start 156.77 47.73) (end 156.77 63.37) (width 1) (layer "F.Cu") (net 1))
 (segment (start 146.51 66.77) (end 145.2 65.46) (width 1) (layer "F.Cu") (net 1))
 (segment (start 145.2 68.87) (end 144.49 69.58) (width 1) (layer "F.Cu") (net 1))
 (segment (start 146.47 63.21) (end 146.47 57.219999) (width 1) (layer "F.Cu") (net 2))
 (segment (start 146.47 57.219999) (end 146.450001 57.2) (width 1) (layer "F.Cu") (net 2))
 (segment (start 131.79 61.695) (end 131.815 61.67) (width 1) (layer "F.Cu") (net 7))
 (segment (start 129.31 60.81) (end 130.17 61.67) (width 1) (layer "F.Cu") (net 7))
 (segment (start 129.31 25.05) (end 129.31 60.81) (width 1) (layer "F.Cu") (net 7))
 (segment (start 131.79 69.58) (end 131.79 61.695) (width 1) (layer "F.Cu") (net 7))
 (segment (start 130.29 24.07) (end 129.31 25.05) (width 1) (layer "F.Cu") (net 7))
 (segment (start 130.17 61.67) (end 131.815 61.67) (width 1) (layer "F.Cu") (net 7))
 (segment (start 146.62 38.09) (end 146.7 38.09) (width 1) (layer "F.Cu") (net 8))
 (segment (start 145.44 36.91) (end 146.62 38.09) (width 1) (layer "F.Cu") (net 8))
 (segment (start 135.36 36.91) (end 145.44 36.91) (width 1) (layer "F.Cu") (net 8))
 (segment (start 132.83 34.38) (end 135.36 36.91) (width 1) (layer "F.Cu") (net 8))
 (segment (start 146.7 38.09) (end 146.7 38.17) (width 1) (layer "F.Cu") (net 8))
 (segment (start 146.7 38.17) (end 146.66 38.13) (width 1) (layer "F.Cu") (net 8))
 (segment (start 132.83 24.07) (end 132.83 34.38) (width 1) (layer "F.Cu") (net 8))
 (via (at 146.7 38.09) (size 0.6) (drill 0.3) (layers "F.Cu" "B.Cu") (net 8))
 (segment (start 155.06 49.15) (end 154.255 49.15) (width 1) (layer "B.Cu") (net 8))
 (segment (start 149.39 40.78) (end 154.72 40.78) (width 1) (layer "B.Cu") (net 8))
 (segment (start 156.2 42.26) (end 156.2 48.01) (width 1) (layer "B.Cu") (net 8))
 (segment (start 154.72 40.78) (end 156.2 42.26) (width 1) (layer "B.Cu") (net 8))
 (segment (start 146.7 38.09) (end 149.39 40.78) (width 1) (layer "B.Cu") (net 8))
 (segment (start 156.2 48.01) (end 155.06 49.15) (width 1) (layer "B.Cu") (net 8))
 (segment (start 157.69 40.94) (end 157.69 26.79) (width 1) (layer "F.Cu") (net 9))
 (segment (start 157.69 26.79) (end 156.89 25.99) (width 1) (layer "F.Cu") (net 9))
 (segment (start 135.37 25.38) (end 135.37 24.07) (width 1) (layer "F.Cu") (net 9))
 (segment (start 135.32 25.43) (end 135.37 25.38) (width 1) (layer "F.Cu") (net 9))
 (segment (start 156.89 25.99) (end 135.88 25.99) (width 1) (layer "F.Cu") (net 9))
 (segment (start 135.88 25.99) (end 135.32 25.43) (width 1) (layer "F.Cu") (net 9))
 (via (at 157.69 40.94) (size 0.6) (drill 0.3) (layers "F.Cu" "B.Cu") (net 9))
 (segment (start 157.69 40.94) (end 157.69 50.13) (width 1) (layer "B.Cu") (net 9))
 (segment (start 156.13 51.69) (end 154.255 51.69) (width 1) (layer "B.Cu") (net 9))
 (segment (start 157.69 50.13) (end 156.13 51.69) (width 1) (layer "B.Cu") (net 9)))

